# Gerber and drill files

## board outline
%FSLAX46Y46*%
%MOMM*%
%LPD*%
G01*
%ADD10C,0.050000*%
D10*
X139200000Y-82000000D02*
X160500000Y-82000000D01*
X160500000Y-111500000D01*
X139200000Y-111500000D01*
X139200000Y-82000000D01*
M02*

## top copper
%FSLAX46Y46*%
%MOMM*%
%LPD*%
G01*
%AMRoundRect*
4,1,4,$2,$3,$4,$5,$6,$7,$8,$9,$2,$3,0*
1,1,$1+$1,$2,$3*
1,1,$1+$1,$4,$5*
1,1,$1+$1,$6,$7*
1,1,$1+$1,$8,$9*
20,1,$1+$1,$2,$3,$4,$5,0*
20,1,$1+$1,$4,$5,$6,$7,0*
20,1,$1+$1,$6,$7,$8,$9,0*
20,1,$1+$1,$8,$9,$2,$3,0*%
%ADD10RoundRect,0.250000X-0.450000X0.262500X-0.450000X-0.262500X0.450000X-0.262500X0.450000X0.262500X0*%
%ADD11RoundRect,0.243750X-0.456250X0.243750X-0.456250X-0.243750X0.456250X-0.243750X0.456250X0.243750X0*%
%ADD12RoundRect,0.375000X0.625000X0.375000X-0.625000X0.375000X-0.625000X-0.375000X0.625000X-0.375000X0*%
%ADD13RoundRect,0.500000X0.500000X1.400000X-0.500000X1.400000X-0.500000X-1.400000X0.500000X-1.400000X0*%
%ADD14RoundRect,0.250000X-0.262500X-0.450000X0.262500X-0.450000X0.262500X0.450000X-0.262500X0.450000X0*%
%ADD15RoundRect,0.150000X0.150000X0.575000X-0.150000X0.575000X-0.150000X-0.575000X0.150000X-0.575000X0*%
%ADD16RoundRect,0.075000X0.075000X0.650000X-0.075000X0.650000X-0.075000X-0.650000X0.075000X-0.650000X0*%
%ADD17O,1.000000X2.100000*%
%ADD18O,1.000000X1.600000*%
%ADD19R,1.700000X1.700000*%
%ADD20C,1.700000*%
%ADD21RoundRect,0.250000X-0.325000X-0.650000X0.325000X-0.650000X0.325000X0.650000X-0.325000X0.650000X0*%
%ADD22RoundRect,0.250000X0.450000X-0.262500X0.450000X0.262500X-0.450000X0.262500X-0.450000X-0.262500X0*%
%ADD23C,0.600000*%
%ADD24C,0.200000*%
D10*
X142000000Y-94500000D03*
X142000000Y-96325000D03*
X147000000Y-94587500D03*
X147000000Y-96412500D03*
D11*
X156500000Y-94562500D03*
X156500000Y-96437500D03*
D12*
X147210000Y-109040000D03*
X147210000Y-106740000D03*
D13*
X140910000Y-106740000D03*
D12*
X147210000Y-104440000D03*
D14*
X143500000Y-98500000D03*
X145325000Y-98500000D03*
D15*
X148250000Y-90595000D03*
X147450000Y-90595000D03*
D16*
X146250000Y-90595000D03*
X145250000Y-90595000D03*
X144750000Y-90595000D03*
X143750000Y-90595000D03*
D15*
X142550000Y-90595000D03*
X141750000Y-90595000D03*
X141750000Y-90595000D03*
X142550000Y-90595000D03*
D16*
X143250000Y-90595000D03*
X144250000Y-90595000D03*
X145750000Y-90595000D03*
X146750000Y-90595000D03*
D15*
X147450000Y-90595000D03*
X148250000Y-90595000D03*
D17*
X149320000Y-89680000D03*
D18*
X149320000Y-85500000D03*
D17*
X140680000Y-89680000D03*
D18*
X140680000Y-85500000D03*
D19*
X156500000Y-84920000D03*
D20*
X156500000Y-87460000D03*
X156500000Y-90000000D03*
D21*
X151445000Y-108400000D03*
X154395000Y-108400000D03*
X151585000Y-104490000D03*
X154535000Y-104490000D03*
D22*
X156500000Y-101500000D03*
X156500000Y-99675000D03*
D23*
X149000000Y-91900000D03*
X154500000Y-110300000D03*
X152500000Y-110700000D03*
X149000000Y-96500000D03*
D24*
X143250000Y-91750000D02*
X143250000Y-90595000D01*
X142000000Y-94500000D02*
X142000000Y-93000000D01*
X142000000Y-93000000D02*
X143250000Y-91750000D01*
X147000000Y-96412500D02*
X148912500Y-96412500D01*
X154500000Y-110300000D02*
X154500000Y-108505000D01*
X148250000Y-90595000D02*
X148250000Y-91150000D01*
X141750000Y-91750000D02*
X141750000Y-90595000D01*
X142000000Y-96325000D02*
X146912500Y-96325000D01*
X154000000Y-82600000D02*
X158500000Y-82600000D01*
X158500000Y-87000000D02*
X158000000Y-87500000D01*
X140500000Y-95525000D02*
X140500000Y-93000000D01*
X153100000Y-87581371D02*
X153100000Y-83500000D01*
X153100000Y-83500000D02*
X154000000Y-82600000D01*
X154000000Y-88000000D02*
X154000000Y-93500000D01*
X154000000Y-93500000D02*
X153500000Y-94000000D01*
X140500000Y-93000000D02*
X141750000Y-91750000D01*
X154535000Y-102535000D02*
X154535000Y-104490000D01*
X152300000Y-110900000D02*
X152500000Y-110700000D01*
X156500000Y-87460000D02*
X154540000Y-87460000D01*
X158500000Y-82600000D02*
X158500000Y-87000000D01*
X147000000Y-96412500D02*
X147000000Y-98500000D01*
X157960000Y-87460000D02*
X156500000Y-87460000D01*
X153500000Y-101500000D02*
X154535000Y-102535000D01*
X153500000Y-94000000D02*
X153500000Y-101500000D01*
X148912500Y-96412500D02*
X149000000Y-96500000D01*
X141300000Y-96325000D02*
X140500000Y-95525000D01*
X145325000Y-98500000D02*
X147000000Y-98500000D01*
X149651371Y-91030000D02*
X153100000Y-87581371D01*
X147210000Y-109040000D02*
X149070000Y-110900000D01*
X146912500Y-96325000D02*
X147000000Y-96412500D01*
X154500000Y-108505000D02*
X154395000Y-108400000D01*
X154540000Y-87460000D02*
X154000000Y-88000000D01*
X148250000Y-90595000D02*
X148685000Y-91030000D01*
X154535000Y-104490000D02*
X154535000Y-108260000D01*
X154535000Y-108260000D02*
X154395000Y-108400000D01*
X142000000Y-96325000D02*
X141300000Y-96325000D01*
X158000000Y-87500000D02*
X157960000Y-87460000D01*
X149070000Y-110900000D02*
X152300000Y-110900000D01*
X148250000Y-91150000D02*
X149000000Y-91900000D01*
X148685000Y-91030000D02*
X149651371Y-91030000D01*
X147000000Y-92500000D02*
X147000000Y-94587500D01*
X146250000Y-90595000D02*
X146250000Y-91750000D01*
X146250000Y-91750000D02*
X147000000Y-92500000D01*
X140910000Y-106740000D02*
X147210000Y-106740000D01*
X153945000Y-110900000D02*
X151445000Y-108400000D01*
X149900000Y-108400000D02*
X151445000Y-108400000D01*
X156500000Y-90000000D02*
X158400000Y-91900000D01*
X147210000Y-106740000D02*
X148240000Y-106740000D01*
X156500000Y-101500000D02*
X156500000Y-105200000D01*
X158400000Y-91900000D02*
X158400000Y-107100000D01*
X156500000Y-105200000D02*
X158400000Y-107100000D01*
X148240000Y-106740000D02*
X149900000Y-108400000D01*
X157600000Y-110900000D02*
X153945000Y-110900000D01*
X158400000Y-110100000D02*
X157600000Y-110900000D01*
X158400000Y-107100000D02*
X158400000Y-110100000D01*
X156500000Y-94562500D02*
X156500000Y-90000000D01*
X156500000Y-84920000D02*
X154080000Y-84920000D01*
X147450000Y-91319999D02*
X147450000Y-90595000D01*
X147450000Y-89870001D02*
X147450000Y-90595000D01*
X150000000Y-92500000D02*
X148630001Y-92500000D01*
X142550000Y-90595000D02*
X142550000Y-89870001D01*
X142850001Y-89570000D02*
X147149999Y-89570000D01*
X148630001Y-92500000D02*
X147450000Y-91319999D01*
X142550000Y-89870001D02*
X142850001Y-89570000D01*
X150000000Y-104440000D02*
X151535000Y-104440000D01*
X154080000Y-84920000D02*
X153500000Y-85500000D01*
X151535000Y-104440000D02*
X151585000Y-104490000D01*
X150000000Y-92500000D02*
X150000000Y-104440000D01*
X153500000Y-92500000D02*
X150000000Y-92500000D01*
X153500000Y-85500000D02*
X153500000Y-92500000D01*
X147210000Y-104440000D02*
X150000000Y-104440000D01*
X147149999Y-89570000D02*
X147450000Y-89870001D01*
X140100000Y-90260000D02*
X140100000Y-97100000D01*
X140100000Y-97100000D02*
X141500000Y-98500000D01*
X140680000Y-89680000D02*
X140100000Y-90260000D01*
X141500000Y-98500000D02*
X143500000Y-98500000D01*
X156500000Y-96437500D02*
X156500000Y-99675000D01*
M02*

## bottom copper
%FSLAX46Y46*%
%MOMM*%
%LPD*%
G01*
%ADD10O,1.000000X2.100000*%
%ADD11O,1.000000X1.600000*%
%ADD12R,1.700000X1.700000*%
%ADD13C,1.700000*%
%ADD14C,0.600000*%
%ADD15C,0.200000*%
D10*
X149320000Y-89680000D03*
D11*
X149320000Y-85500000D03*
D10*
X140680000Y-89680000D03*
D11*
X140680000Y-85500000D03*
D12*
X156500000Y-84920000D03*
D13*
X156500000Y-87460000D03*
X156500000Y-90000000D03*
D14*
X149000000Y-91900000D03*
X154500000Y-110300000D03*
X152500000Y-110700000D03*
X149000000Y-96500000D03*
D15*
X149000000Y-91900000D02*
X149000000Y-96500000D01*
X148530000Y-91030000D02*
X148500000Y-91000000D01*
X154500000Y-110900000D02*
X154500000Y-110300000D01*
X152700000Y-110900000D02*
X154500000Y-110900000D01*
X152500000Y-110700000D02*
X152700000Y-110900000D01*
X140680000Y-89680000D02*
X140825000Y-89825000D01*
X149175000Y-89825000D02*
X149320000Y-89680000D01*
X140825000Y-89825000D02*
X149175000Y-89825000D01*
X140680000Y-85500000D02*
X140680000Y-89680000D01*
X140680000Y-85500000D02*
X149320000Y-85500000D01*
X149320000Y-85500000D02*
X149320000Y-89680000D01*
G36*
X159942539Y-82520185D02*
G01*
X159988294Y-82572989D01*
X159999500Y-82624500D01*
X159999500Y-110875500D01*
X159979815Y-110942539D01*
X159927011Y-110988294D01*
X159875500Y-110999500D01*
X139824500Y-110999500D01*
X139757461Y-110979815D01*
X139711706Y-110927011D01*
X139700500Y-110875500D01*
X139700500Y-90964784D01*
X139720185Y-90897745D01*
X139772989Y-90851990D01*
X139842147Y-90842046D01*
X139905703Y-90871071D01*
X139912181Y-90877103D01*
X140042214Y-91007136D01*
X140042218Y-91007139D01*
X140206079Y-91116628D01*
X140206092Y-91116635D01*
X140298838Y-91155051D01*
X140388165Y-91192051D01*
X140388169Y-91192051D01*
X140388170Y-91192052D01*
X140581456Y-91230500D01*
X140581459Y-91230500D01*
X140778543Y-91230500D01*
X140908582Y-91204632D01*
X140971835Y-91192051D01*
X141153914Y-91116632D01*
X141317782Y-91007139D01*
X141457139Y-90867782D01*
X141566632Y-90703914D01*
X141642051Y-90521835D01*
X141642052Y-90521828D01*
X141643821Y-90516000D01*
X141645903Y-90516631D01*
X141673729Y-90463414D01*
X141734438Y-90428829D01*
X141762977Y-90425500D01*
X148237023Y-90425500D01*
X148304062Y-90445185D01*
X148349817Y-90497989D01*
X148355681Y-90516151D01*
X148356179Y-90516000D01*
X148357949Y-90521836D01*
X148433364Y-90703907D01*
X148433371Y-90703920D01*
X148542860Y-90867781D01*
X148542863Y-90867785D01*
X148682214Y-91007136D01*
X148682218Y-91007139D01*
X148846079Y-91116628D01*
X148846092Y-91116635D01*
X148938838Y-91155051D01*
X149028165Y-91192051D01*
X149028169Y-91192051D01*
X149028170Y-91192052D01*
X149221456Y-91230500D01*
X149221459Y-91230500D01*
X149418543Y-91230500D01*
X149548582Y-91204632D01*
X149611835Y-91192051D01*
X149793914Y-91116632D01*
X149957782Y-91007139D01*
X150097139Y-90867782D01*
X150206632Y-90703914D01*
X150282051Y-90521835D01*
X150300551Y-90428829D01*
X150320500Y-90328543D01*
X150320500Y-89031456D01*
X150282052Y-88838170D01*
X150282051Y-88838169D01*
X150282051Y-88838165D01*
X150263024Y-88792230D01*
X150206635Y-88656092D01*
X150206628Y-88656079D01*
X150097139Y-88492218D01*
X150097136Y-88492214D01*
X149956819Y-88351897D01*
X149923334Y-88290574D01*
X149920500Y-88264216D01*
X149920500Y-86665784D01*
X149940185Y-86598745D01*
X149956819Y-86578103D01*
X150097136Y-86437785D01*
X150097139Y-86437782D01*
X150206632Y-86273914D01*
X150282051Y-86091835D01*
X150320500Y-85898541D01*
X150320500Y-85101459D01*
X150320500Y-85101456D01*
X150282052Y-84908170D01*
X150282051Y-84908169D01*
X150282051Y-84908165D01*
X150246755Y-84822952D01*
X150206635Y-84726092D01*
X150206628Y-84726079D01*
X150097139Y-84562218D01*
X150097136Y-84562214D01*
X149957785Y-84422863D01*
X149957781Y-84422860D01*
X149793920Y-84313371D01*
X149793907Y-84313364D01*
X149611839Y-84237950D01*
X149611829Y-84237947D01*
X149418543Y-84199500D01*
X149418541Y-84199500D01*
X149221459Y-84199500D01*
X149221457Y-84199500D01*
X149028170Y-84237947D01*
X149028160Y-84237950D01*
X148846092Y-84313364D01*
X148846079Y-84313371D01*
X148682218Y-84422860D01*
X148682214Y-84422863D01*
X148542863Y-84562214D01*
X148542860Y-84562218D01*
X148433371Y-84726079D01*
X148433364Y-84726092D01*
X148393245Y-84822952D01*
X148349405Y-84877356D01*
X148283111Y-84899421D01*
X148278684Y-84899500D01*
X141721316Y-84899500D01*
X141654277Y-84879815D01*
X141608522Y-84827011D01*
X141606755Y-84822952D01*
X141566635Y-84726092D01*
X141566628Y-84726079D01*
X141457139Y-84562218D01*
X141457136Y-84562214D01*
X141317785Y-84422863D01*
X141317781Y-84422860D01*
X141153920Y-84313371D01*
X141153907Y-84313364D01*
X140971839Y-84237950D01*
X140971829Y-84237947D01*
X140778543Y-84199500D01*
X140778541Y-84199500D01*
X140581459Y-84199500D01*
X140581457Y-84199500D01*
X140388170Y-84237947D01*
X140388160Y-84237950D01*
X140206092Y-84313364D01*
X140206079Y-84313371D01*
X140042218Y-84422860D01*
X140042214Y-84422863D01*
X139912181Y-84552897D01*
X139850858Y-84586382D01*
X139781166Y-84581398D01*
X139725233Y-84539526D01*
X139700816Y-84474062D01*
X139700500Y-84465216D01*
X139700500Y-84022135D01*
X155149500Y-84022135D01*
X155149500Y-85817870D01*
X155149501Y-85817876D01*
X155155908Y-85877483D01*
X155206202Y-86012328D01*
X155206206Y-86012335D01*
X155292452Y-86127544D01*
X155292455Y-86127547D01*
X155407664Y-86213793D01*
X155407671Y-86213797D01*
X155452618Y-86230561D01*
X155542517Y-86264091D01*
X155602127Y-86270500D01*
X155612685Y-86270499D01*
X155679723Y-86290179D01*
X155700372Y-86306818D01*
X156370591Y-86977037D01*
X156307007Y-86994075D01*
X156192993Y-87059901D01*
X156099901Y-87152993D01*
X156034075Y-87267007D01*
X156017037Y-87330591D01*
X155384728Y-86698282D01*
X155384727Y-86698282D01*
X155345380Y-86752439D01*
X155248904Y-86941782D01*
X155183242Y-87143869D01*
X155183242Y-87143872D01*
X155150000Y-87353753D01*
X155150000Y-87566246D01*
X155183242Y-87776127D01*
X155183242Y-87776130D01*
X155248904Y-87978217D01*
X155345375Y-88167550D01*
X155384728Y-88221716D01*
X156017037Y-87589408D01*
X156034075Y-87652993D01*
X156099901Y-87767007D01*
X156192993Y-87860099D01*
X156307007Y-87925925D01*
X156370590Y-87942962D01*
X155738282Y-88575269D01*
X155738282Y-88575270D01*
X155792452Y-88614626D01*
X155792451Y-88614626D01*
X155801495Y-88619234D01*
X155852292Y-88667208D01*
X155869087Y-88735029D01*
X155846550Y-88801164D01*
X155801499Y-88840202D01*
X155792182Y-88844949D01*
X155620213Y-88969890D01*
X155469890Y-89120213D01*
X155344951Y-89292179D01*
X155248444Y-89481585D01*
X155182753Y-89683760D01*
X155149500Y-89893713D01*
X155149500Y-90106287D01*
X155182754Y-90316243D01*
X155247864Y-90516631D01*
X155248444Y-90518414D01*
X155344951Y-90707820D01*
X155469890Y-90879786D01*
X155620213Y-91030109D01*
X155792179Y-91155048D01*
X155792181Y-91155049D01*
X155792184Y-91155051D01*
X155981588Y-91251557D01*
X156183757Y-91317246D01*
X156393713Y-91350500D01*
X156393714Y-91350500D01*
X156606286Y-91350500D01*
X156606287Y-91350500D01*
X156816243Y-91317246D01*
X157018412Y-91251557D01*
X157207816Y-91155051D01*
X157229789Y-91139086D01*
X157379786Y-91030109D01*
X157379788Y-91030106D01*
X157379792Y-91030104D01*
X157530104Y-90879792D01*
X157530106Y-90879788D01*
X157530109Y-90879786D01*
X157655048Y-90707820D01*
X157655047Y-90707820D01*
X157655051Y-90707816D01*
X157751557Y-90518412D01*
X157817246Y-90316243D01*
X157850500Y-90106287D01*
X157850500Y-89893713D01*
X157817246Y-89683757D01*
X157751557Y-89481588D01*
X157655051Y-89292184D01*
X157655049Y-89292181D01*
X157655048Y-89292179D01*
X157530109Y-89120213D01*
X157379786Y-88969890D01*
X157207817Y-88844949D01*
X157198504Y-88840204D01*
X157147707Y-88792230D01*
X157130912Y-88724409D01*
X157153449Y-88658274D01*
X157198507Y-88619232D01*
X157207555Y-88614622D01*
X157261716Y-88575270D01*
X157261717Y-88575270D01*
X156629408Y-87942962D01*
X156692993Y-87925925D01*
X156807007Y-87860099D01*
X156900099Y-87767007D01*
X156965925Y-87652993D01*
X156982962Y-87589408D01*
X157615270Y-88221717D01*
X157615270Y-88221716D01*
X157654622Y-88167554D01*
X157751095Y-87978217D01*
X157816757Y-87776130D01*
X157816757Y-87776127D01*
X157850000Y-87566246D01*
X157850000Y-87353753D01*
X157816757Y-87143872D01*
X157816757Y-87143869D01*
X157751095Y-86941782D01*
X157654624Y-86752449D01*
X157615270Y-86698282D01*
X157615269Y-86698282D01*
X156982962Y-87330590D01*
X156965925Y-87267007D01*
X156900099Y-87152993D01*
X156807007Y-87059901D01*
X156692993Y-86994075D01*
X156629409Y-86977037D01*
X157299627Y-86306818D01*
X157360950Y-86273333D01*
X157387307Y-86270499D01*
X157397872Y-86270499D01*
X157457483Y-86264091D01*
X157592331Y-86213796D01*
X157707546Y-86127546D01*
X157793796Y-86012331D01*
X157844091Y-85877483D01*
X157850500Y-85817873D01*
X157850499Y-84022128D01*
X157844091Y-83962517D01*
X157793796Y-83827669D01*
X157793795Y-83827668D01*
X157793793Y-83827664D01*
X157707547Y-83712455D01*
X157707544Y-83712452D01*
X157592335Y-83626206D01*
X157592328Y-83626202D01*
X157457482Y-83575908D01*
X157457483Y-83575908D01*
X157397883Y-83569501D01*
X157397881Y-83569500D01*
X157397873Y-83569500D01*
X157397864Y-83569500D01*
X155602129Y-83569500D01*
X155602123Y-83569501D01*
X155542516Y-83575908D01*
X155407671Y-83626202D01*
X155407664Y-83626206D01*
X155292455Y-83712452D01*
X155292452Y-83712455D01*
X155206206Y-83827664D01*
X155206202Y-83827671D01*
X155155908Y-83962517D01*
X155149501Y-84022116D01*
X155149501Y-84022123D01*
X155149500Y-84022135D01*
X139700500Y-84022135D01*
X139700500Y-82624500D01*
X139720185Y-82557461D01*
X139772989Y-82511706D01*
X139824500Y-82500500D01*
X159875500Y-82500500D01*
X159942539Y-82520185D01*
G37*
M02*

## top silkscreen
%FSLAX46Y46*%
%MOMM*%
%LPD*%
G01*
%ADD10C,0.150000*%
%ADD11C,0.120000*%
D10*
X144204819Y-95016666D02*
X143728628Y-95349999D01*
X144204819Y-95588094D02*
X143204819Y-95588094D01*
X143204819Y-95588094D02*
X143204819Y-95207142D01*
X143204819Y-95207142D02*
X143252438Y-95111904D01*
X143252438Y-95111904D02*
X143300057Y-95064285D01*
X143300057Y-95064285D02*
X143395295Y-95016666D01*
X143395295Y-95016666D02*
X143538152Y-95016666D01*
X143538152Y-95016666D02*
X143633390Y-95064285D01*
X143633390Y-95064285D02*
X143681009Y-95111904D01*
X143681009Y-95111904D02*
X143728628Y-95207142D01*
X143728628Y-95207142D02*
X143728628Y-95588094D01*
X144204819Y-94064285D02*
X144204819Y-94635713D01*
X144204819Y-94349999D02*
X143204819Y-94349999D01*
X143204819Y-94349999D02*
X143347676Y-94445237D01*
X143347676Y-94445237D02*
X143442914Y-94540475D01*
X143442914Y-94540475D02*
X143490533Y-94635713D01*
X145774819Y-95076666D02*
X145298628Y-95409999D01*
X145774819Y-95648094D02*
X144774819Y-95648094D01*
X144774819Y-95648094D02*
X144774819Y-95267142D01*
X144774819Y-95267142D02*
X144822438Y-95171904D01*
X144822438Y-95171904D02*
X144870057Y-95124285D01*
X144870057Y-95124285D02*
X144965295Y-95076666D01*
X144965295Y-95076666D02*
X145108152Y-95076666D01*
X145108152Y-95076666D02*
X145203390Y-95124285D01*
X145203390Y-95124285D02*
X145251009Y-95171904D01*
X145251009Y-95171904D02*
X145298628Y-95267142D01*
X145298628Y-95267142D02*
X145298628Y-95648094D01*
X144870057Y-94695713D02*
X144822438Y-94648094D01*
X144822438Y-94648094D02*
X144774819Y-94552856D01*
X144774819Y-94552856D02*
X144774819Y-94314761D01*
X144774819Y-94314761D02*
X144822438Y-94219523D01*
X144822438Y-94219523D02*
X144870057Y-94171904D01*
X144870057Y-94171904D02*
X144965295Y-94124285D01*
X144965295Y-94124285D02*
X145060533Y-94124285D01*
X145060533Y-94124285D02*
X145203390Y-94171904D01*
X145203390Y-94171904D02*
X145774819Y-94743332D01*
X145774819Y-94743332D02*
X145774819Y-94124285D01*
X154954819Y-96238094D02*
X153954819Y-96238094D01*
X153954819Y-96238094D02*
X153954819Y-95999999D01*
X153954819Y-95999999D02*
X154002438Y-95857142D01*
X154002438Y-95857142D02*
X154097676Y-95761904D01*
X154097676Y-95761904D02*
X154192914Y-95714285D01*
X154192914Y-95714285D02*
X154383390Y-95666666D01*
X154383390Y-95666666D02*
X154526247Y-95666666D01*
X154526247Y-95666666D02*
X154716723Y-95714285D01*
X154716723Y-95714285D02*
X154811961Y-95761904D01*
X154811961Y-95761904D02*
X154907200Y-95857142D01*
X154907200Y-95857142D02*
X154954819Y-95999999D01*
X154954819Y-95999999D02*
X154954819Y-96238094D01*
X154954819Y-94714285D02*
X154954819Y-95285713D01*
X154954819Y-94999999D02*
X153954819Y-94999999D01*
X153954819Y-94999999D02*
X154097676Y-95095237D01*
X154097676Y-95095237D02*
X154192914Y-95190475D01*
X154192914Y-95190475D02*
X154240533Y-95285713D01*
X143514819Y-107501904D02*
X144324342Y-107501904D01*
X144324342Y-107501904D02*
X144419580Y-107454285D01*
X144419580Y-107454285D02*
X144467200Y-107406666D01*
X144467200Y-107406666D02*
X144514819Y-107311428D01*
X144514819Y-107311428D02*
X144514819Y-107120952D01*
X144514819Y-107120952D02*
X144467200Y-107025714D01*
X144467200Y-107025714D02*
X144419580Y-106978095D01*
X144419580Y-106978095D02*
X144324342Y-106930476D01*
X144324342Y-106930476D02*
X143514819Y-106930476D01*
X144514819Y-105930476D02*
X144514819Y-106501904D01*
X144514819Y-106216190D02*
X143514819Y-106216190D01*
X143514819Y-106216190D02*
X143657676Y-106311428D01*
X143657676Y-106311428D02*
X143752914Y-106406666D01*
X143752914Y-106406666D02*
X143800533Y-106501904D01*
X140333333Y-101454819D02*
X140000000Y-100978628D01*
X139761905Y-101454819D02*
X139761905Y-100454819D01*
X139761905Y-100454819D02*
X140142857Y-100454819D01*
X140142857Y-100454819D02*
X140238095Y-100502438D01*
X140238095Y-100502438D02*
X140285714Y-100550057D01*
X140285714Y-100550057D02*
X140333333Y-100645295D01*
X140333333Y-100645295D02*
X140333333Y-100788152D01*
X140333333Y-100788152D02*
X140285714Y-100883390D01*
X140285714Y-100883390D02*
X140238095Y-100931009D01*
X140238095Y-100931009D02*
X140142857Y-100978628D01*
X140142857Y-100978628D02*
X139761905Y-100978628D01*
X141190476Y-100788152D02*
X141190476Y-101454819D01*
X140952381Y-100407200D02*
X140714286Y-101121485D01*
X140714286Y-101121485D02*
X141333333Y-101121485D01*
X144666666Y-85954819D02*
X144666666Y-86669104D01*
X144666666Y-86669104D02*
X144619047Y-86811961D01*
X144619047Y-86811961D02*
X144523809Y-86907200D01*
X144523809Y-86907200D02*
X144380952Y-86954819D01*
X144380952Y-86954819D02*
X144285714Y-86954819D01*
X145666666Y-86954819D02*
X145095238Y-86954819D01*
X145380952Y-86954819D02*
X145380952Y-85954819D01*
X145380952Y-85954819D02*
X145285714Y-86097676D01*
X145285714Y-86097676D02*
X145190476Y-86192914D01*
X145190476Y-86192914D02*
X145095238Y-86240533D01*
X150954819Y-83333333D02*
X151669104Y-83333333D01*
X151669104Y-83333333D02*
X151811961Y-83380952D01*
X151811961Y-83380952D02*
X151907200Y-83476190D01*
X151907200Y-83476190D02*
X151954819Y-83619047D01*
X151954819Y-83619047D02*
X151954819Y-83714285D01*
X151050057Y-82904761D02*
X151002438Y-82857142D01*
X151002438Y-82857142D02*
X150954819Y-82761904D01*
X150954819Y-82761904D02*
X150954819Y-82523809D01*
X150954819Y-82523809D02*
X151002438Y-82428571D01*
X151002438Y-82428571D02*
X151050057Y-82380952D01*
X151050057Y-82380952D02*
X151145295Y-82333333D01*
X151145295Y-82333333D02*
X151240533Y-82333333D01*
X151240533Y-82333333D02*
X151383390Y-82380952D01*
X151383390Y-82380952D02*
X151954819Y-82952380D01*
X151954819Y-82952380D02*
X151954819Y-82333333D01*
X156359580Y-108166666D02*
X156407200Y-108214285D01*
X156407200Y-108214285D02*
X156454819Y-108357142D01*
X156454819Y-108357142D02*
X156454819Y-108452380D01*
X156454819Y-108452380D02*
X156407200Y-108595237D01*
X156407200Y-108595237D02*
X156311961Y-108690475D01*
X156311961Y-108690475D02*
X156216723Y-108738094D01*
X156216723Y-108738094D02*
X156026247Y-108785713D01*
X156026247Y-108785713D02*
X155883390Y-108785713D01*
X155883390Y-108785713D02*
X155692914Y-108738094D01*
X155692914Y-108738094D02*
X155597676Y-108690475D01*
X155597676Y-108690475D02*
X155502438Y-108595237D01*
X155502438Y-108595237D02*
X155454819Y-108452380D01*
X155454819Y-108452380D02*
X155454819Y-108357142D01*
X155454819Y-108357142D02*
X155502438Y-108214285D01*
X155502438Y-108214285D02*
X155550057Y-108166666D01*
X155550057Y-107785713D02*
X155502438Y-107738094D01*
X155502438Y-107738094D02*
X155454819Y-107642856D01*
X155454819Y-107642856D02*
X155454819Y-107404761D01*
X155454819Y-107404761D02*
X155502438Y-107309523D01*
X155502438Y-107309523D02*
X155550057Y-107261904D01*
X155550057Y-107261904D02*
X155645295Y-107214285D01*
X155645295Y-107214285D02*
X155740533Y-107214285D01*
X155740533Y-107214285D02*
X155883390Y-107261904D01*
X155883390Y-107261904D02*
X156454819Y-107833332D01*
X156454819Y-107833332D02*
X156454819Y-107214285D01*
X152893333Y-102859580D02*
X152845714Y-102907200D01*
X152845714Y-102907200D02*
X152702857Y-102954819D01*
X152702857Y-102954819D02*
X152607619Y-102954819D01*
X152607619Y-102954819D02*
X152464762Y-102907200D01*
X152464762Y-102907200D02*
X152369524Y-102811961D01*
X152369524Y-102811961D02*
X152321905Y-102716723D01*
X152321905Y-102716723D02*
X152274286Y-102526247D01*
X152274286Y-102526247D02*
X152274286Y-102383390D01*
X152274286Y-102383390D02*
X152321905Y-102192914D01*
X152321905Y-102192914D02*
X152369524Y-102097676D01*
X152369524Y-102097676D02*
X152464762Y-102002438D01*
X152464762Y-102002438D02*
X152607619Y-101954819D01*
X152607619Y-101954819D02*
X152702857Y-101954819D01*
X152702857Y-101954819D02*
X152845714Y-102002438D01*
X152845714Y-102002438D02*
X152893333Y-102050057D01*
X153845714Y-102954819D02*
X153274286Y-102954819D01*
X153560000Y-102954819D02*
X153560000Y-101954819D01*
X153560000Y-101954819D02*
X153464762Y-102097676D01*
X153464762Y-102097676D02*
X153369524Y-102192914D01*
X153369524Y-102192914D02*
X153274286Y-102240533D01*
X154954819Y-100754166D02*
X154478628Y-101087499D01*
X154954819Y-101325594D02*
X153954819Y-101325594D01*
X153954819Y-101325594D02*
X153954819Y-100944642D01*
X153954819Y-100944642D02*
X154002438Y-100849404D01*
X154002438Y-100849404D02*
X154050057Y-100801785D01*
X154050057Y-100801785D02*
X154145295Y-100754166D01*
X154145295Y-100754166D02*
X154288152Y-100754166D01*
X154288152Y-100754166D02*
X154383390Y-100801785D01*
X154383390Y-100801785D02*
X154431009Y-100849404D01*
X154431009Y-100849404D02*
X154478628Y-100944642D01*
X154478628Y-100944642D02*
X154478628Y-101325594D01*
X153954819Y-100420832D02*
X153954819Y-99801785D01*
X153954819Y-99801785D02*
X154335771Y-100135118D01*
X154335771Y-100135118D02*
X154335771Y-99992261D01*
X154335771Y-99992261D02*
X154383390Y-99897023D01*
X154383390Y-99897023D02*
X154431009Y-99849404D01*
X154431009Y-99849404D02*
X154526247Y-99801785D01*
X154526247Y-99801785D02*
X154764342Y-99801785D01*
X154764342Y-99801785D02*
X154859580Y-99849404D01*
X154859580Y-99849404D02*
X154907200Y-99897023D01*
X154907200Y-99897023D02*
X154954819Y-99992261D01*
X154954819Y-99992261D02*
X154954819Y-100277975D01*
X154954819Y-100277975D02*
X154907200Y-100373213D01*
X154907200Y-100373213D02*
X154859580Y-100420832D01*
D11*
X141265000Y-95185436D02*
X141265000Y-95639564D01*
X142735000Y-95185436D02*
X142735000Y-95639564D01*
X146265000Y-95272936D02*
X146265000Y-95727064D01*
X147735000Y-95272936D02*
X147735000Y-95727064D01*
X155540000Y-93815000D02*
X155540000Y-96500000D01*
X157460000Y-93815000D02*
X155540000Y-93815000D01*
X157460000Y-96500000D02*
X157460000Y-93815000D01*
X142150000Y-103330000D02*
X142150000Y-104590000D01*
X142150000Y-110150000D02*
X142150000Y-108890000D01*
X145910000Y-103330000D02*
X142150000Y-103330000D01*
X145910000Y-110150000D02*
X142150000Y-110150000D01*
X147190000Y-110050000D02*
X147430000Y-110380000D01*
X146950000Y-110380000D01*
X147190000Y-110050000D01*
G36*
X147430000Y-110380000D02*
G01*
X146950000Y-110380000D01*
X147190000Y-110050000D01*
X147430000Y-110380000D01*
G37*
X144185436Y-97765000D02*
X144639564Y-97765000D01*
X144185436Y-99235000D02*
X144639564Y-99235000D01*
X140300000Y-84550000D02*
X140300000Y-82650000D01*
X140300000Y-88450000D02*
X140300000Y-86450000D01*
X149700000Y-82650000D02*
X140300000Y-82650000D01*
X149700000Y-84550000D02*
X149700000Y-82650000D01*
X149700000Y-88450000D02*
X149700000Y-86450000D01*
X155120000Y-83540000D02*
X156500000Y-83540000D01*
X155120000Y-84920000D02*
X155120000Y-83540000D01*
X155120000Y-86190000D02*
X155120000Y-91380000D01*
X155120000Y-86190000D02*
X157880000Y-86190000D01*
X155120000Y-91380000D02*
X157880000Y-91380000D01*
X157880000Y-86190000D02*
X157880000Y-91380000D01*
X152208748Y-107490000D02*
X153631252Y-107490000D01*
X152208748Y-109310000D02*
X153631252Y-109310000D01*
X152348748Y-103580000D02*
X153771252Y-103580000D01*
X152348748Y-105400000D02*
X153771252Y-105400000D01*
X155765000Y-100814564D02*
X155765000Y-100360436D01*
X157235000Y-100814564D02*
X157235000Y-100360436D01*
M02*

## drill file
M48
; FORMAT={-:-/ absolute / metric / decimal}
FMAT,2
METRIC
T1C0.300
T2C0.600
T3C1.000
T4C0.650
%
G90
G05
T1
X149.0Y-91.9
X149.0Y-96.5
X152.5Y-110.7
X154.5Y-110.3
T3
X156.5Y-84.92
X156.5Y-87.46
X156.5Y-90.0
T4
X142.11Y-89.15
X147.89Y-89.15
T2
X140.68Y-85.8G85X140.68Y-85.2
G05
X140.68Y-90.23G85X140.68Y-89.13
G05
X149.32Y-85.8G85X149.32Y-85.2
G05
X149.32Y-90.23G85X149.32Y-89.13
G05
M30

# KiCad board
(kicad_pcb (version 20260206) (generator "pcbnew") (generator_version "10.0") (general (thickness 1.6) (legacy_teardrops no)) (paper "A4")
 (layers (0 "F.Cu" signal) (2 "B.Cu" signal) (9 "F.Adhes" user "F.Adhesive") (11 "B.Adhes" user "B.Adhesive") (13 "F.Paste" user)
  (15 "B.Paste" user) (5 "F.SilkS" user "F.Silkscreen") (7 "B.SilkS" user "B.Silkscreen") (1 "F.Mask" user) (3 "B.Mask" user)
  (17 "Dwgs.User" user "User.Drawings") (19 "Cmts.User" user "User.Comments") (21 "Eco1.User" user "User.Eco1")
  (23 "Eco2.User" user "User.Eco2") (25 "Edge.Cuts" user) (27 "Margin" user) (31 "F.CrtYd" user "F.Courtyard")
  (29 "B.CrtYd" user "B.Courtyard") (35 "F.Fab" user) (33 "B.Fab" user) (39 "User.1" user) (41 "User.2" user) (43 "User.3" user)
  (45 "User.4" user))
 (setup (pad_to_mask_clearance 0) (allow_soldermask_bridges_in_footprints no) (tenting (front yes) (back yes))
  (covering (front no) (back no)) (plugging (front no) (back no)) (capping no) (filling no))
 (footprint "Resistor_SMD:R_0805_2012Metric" (layer "F.Cu") (at 142 95.4125 -90)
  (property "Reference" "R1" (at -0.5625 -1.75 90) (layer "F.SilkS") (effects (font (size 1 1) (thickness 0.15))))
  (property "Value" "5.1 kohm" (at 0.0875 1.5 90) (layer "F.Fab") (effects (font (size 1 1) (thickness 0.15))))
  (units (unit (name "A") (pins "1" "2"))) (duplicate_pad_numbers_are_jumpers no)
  (fp_line (start -0.227064 0.735) (end 0.227064 0.735) (stroke (width 0.12) (type solid)) (layer "F.SilkS"))
  (fp_line (start -0.227064 -0.735) (end 0.227064 -0.735) (stroke (width 0.12) (type solid)) (layer "F.SilkS"))
  (pad "1" smd roundrect (at -0.9125 0 270) (size 1.025 1.4) (layers "F.Cu" "F.Mask" "F.Paste") (roundrect_rratio 0.243902)
   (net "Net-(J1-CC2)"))
  (pad "2" smd roundrect (at 0.9125 0 270) (size 1.025 1.4) (layers "F.Cu" "F.Mask" "F.Paste") (roundrect_rratio 0.243902) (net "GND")))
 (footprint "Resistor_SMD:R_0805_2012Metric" (layer "F.Cu") (at 147 95.5 -90)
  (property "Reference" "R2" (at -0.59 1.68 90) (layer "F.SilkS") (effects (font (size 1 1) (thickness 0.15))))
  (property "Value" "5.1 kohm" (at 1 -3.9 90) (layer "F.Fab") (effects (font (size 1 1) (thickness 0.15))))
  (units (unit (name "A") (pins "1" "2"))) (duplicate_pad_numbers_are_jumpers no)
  (fp_line (start -0.227064 0.735) (end 0.227064 0.735) (stroke (width 0.12) (type solid)) (layer "F.SilkS"))
  (fp_line (start -0.227064 -0.735) (end 0.227064 -0.735) (stroke (width 0.12) (type solid)) (layer "F.SilkS"))
  (pad "1" smd roundrect (at -0.9125 0 270) (size 1.025 1.4) (layers "F.Cu" "F.Mask" "F.Paste") (roundrect_rratio 0.243902)
   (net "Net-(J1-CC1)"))
  (pad "2" smd roundrect (at 0.9125 0 270) (size 1.025 1.4) (layers "F.Cu" "F.Mask" "F.Paste") (roundrect_rratio 0.243902) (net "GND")))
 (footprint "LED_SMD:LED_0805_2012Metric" (layer "F.Cu") (at 156.5 95.5 -90)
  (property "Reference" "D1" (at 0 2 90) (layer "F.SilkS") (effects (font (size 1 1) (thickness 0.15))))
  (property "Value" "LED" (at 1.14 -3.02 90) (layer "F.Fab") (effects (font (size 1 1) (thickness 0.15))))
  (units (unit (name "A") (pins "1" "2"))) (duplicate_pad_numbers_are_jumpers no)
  (fp_line (start -1.685 0.96) (end 1 0.96) (stroke (width 0.12) (type solid)) (layer "F.SilkS"))
  (fp_line (start -1.685 -0.96) (end -1.685 0.96) (stroke (width 0.12) (type solid)) (layer "F.SilkS"))
  (fp_line (start 1 -0.96) (end -1.685 -0.96) (stroke (width 0.12) (type solid)) (layer "F.SilkS"))
  (pad "1" smd roundrect (at -0.9375 0 270) (size 0.975 1.4) (layers "F.Cu" "F.Mask" "F.Paste") (roundrect_rratio 0.25) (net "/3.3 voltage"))
  (pad "2" smd roundrect (at 0.9375 0 270) (size 0.975 1.4) (layers "F.Cu" "F.Mask" "F.Paste") (roundrect_rratio 0.25) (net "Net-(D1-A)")))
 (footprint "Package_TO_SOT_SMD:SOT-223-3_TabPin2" (layer "F.Cu") (at 144.06 106.74 180)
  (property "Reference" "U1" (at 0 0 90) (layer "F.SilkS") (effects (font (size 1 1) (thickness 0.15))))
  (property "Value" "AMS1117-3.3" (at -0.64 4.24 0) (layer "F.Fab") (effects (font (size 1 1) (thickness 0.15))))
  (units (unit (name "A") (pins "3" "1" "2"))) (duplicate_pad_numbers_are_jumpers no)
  (fp_line (start 1.91 3.41) (end 1.91 2.15) (stroke (width 0.12) (type solid)) (layer "F.SilkS"))
  (fp_line (start 1.91 -3.41) (end 1.91 -2.15) (stroke (width 0.12) (type solid)) (layer "F.SilkS"))
  (fp_line (start -1.85 3.41) (end 1.91 3.41) (stroke (width 0.12) (type solid)) (layer "F.SilkS"))
  (fp_line (start -1.85 -3.41) (end 1.91 -3.41) (stroke (width 0.12) (type solid)) (layer "F.SilkS"))
  (fp_poly
   (pts (xy -3.13 -3.31) (xy -3.37 -3.64) (xy -2.89 -3.64) (xy -3.13 -3.31)) (stroke (width 0.12) (type solid)) (fill yes) (layer "F.SilkS"))
  (pad "1" smd roundrect (at -3.15 -2.3 180) (size 2 1.5) (layers "F.Cu" "F.Mask" "F.Paste") (roundrect_rratio 0.25) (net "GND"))
  (pad "2" smd roundrect (at -3.15 0 180) (size 2 1.5) (layers "F.Cu" "F.Mask" "F.Paste") (roundrect_rratio 0.25) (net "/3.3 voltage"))
  (pad "2" smd roundrect (at 3.15 0 180) (size 2 3.8) (layers "F.Cu" "F.Mask" "F.Paste") (roundrect_rratio 0.25) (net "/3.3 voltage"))
  (pad "3" smd roundrect (at -3.15 2.3 180) (size 2 1.5) (layers "F.Cu" "F.Mask" "F.Paste") (roundrect_rratio 0.25) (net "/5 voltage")))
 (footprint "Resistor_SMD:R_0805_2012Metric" (layer "F.Cu") (at 144.4125 98.5)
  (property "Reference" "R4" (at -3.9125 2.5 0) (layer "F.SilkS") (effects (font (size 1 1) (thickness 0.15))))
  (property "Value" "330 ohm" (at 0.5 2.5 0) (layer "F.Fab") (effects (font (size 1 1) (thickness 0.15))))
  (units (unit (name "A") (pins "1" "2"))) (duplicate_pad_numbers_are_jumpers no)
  (fp_line (start -0.227064 -0.735) (end 0.227064 -0.735) (stroke (width 0.12) (type solid)) (layer "F.SilkS"))
  (fp_line (start -0.227064 0.735) (end 0.227064 0.735) (stroke (width 0.12) (type solid)) (layer "F.SilkS"))
  (pad "1" smd roundrect (at -0.9125 0) (size 1.025 1.4) (layers "F.Cu" "F.Mask" "F.Paste") (roundrect_rratio 0.243902)
   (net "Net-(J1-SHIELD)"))
  (pad "2" smd roundrect (at 0.9125 0) (size 1.025 1.4) (layers "F.Cu" "F.Mask" "F.Paste") (roundrect_rratio 0.243902) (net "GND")))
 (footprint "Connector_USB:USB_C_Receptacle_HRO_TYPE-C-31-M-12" (layer "F.Cu") (at 145 86.55 180)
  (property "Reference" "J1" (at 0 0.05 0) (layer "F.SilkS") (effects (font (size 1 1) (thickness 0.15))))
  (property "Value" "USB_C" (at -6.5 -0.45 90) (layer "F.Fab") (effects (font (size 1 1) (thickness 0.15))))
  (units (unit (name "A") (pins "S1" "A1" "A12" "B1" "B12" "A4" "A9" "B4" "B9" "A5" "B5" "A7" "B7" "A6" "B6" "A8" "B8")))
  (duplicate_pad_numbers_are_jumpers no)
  (fp_line (start 4.7 2) (end 4.7 3.9) (stroke (width 0.12) (type solid)) (layer "F.SilkS"))
  (fp_line (start 4.7 -1.9) (end 4.7 0.1) (stroke (width 0.12) (type solid)) (layer "F.SilkS"))
  (fp_line (start -4.7 3.9) (end 4.7 3.9) (stroke (width 0.12) (type solid)) (layer "F.SilkS"))
  (fp_line (start -4.7 2) (end -4.7 3.9) (stroke (width 0.12) (type solid)) (layer "F.SilkS"))
  (fp_line (start -4.7 -1.9) (end -4.7 0.1) (stroke (width 0.12) (type solid)) (layer "F.SilkS"))
  (pad "" np_thru_hole circle (at -2.89 -2.6 180) (size 0.65 0.65) (drill 0.65) (layers "*.Cu" "*.Mask"))
  (pad "" np_thru_hole circle (at 2.89 -2.6 180) (size 0.65 0.65) (drill 0.65) (layers "*.Cu" "*.Mask"))
  (pad "A1" smd roundrect (at -3.25 -4.045 180) (size 0.6 1.45) (layers "F.Cu" "F.Mask" "F.Paste") (roundrect_rratio 0.25) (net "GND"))
  (pad "A4" smd roundrect (at -2.45 -4.045 180) (size 0.6 1.45) (layers "F.Cu" "F.Mask" "F.Paste") (roundrect_rratio 0.25)
   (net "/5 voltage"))
  (pad "A5" smd roundrect (at -1.25 -4.045 180) (size 0.3 1.45) (layers "F.Cu" "F.Mask" "F.Paste") (roundrect_rratio 0.25)
   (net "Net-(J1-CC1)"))
  (pad "A6" smd roundrect (at -0.25 -4.045 180) (size 0.3 1.45) (layers "F.Cu" "F.Mask" "F.Paste") (roundrect_rratio 0.25)
   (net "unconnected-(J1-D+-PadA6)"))
  (pad "A7" smd roundrect (at 0.25 -4.045 180) (size 0.3 1.45) (layers "F.Cu" "F.Mask" "F.Paste") (roundrect_rratio 0.25)
   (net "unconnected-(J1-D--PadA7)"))
  (pad "A8" smd roundrect (at 1.25 -4.045 180) (size 0.3 1.45) (layers "F.Cu" "F.Mask" "F.Paste") (roundrect_rratio 0.25)
   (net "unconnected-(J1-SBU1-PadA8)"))
  (pad "A9" smd roundrect (at 2.45 -4.045 180) (size 0.6 1.45) (layers "F.Cu" "F.Mask" "F.Paste") (roundrect_rratio 0.25) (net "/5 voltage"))
  (pad "A12" smd roundrect (at 3.25 -4.045 180) (size 0.6 1.45) (layers "F.Cu" "F.Mask" "F.Paste") (roundrect_rratio 0.25) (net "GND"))
  (pad "B1" smd roundrect (at 3.25 -4.045 180) (size 0.6 1.45) (layers "F.Cu" "F.Mask" "F.Paste") (roundrect_rratio 0.25) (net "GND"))
  (pad "B4" smd roundrect (at 2.45 -4.045 180) (size 0.6 1.45) (layers "F.Cu" "F.Mask" "F.Paste") (roundrect_rratio 0.25) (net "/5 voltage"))
  (pad "B5" smd roundrect (at 1.75 -4.045 180) (size 0.3 1.45) (layers "F.Cu" "F.Mask" "F.Paste") (roundrect_rratio 0.25)
   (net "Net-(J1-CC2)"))
  (pad "B6" smd roundrect (at 0.75 -4.045 180) (size 0.3 1.45) (layers "F.Cu" "F.Mask" "F.Paste") (roundrect_rratio 0.25)
   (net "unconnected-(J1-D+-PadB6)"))
  (pad "B7" smd roundrect (at -0.75 -4.045 180) (size 0.3 1.45) (layers "F.Cu" "F.Mask" "F.Paste") (roundrect_rratio 0.25)
   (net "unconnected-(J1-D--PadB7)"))
  (pad "B8" smd roundrect (at -1.75 -4.045 180) (size 0.3 1.45) (layers "F.Cu" "F.Mask" "F.Paste") (roundrect_rratio 0.25)
   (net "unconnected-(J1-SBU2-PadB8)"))
  (pad "B9" smd roundrect (at -2.45 -4.045 180) (size 0.6 1.45) (layers "F.Cu" "F.Mask" "F.Paste") (roundrect_rratio 0.25)
   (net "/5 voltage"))
  (pad "B12" smd roundrect (at -3.25 -4.045 180) (size 0.6 1.45) (layers "F.Cu" "F.Mask" "F.Paste") (roundrect_rratio 0.25) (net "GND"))
  (pad "SH" thru_hole oval (at -4.32 -3.13 180) (size 1 2.1) (drill oval 0.6 1.7) (layers "*.Cu" "*.Mask") (remove_unused_layers no)
   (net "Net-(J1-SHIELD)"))
  (pad "SH" thru_hole oval (at -4.32 1.05 180) (size 1 1.6) (drill oval 0.6 1.2) (layers "*.Cu" "*.Mask") (remove_unused_layers no)
   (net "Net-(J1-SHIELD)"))
  (pad "SH" thru_hole oval (at 4.32 -3.13 180) (size 1 2.1) (drill oval 0.6 1.7) (layers "*.Cu" "*.Mask") (remove_unused_layers no)
   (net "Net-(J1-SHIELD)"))
  (pad "SH" thru_hole oval (at 4.32 1.05 180) (size 1 1.6) (drill oval 0.6 1.2) (layers "*.Cu" "*.Mask") (remove_unused_layers no)
   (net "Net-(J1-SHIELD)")))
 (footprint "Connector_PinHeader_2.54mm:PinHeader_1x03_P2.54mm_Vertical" (layer "F.Cu") (at 156.5 84.92)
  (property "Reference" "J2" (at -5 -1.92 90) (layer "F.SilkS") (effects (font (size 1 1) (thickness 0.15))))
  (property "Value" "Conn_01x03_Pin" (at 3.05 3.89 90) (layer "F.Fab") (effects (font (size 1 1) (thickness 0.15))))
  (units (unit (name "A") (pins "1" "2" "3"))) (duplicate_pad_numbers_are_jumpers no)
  (fp_line (start -1.38 -1.38) (end 0 -1.38) (stroke (width 0.12) (type solid)) (layer "F.SilkS"))
  (fp_line (start -1.38 0) (end -1.38 -1.38) (stroke (width 0.12) (type solid)) (layer "F.SilkS"))
  (fp_line (start -1.38 1.27) (end -1.38 6.46) (stroke (width 0.12) (type solid)) (layer "F.SilkS"))
  (fp_line (start -1.38 1.27) (end 1.38 1.27) (stroke (width 0.12) (type solid)) (layer "F.SilkS"))
  (fp_line (start -1.38 6.46) (end 1.38 6.46) (stroke (width 0.12) (type solid)) (layer "F.SilkS"))
  (fp_line (start 1.38 1.27) (end 1.38 6.46) (stroke (width 0.12) (type solid)) (layer "F.SilkS"))
  (pad "1" thru_hole rect (at 0 0) (size 1.7 1.7) (drill 1) (layers "*.Cu" "*.Mask") (remove_unused_layers no) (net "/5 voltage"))
  (pad "2" thru_hole circle (at 0 2.54) (size 1.7 1.7) (drill 1) (layers "*.Cu" "*.Mask") (remove_unused_layers no) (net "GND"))
  (pad "3" thru_hole circle (at 0 5.08) (size 1.7 1.7) (drill 1) (layers "*.Cu" "*.Mask") (remove_unused_layers no) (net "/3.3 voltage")))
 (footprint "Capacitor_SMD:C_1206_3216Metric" (layer "F.Cu") (at 152.92 108.4)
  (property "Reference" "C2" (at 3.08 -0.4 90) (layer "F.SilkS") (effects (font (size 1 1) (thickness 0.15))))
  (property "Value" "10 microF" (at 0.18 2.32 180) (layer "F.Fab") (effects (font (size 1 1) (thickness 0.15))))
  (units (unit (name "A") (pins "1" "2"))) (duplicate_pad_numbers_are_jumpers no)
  (fp_line (start -0.711252 -0.91) (end 0.711252 -0.91) (stroke (width 0.12) (type solid)) (layer "F.SilkS"))
  (fp_line (start -0.711252 0.91) (end 0.711252 0.91) (stroke (width 0.12) (type solid)) (layer "F.SilkS"))
  (pad "1" smd roundrect (at -1.475 0) (size 1.15 1.8) (layers "F.Cu" "F.Mask" "F.Paste") (roundrect_rratio 0.217391) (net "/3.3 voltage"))
  (pad "2" smd roundrect (at 1.475 0) (size 1.15 1.8) (layers "F.Cu" "F.Mask" "F.Paste") (roundrect_rratio 0.217391) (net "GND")))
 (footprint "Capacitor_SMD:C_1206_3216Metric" (layer "F.Cu") (at 153.06 104.49)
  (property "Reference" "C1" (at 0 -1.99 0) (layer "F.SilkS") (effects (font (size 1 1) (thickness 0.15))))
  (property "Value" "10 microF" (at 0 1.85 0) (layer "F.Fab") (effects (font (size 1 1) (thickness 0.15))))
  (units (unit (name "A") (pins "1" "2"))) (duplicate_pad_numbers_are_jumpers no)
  (fp_line (start -0.711252 -0.91) (end 0.711252 -0.91) (stroke (width 0.12) (type solid)) (layer "F.SilkS"))
  (fp_line (start -0.711252 0.91) (end 0.711252 0.91) (stroke (width 0.12) (type solid)) (layer "F.SilkS"))
  (pad "1" smd roundrect (at -1.475 0) (size 1.15 1.8) (layers "F.Cu" "F.Mask" "F.Paste") (roundrect_rratio 0.217391) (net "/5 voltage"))
  (pad "2" smd roundrect (at 1.475 0) (size 1.15 1.8) (layers "F.Cu" "F.Mask" "F.Paste") (roundrect_rratio 0.217391) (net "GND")))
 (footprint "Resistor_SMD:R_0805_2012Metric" (layer "F.Cu") (at 156.5 100.5875 90)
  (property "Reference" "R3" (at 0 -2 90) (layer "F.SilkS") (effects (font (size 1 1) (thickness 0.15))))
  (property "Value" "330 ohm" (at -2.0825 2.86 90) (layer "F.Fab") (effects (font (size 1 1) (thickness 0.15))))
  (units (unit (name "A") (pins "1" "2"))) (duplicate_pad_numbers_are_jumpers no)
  (fp_line (start -0.227064 -0.735) (end 0.227064 -0.735) (stroke (width 0.12) (type solid)) (layer "F.SilkS"))
  (fp_line (start -0.227064 0.735) (end 0.227064 0.735) (stroke (width 0.12) (type solid)) (layer "F.SilkS"))
  (pad "1" smd roundrect (at -0.9125 0 90) (size 1.025 1.4) (layers "F.Cu" "F.Mask" "F.Paste") (roundrect_rratio 0.243902)
   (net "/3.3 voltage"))
  (pad "2" smd roundrect (at 0.9125 0 90) (size 1.025 1.4) (layers "F.Cu" "F.Mask" "F.Paste") (roundrect_rratio 0.243902) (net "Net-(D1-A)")))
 (gr_rect (start 139.2 82) (end 160.5 111.5) (stroke (width 0.05) (type default)) (fill no) (layer "Edge.Cuts"))
 (segment (start 143.25 91.75) (end 143.25 90.595) (width 0.2) (layer "F.Cu") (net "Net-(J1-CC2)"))
 (segment (start 142 94.5) (end 142 93) (width 0.2) (layer "F.Cu") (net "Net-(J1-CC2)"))
 (segment (start 142 93) (end 143.25 91.75) (width 0.2) (layer "F.Cu") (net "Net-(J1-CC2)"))
 (segment (start 147 96.4125) (end 148.9125 96.4125) (width 0.2) (layer "F.Cu") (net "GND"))
 (segment (start 154.5 110.3) (end 154.5 108.505) (width 0.2) (layer "F.Cu") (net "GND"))
 (segment (start 148.25 90.595) (end 148.25 91.15) (width 0.2) (layer "F.Cu") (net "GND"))
 (segment (start 141.75 91.75) (end 141.75 90.595) (width 0.2) (layer "F.Cu") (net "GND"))
 (segment (start 142 96.325) (end 146.9125 96.325) (width 0.2) (layer "F.Cu") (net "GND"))
 (segment (start 154 82.6) (end 158.5 82.6) (width 0.2) (layer "F.Cu") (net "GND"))
 (segment (start 158.5 87) (end 158 87.5) (width 0.2) (layer "F.Cu") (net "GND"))
 (segment (start 140.5 95.525) (end 140.5 93) (width 0.2) (layer "F.Cu") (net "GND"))
 (segment (start 153.1 87.581371) (end 153.1 83.5) (width 0.2) (layer "F.Cu") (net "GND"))
 (segment (start 153.1 83.5) (end 154 82.6) (width 0.2) (layer "F.Cu") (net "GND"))
 (segment (start 154 88) (end 154 93.5) (width 0.2) (layer "F.Cu") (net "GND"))
 (segment (start 154 93.5) (end 153.5 94) (width 0.2) (layer "F.Cu") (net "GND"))
 (segment (start 140.5 93) (end 141.75 91.75) (width 0.2) (layer "F.Cu") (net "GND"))
 (segment (start 154.535 102.535) (end 154.535 104.49) (width 0.2) (layer "F.Cu") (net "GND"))
 (segment (start 152.3 110.9) (end 152.5 110.7) (width 0.2) (layer "F.Cu") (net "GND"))
 (segment (start 156.5 87.46) (end 154.54 87.46) (width 0.2) (layer "F.Cu") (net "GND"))
 (segment (start 158.5 82.6) (end 158.5 87) (width 0.2) (layer "F.Cu") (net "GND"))
 (segment (start 147 96.4125) (end 147 98.5) (width 0.2) (layer "F.Cu") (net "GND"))
 (segment (start 157.96 87.46) (end 156.5 87.46) (width 0.2) (layer "F.Cu") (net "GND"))
 (segment (start 153.5 101.5) (end 154.535 102.535) (width 0.2) (layer "F.Cu") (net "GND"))
 (segment (start 153.5 94) (end 153.5 101.5) (width 0.2) (layer "F.Cu") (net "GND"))
 (segment (start 148.9125 96.4125) (end 149 96.5) (width 0.2) (layer "F.Cu") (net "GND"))
 (segment (start 141.3 96.325) (end 140.5 95.525) (width 0.2) (layer "F.Cu") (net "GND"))
 (segment (start 145.325 98.5) (end 147 98.5) (width 0.2) (layer "F.Cu") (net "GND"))
 (segment (start 149.651371 91.03) (end 153.1 87.581371) (width 0.2) (layer "F.Cu") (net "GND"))
 (segment (start 147.21 109.04) (end 149.07 110.9) (width 0.2) (layer "F.Cu") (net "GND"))
 (segment (start 146.9125 96.325) (end 147 96.4125) (width 0.2) (layer "F.Cu") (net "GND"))
 (segment (start 154.5 108.505) (end 154.395 108.4) (width 0.2) (layer "F.Cu") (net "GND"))
 (segment (start 154.54 87.46) (end 154 88) (width 0.2) (layer "F.Cu") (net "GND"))
 (segment (start 148.25 90.595) (end 148.685 91.03) (width 0.2) (layer "F.Cu") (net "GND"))
 (segment (start 154.535 104.49) (end 154.535 108.26) (width 0.2) (layer "F.Cu") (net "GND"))
 (segment (start 154.535 108.26) (end 154.395 108.4) (width 0.2) (layer "F.Cu") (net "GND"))
 (segment (start 142 96.325) (end 141.3 96.325) (width 0.2) (layer "F.Cu") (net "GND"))
 (segment (start 158 87.5) (end 157.96 87.46) (width 0.2) (layer "F.Cu") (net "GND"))
 (segment (start 149.07 110.9) (end 152.3 110.9) (width 0.2) (layer "F.Cu") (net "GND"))
 (segment (start 148.25 91.15) (end 149 91.9) (width 0.2) (layer "F.Cu") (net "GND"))
 (segment (start 148.685 91.03) (end 149.651371 91.03) (width 0.2) (layer "F.Cu") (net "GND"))
 (via (at 149 91.9) (size 0.6) (drill 0.3) (layers "F.Cu" "B.Cu") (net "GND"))
 (via (at 154.5 110.3) (size 0.6) (drill 0.3) (layers "F.Cu" "B.Cu") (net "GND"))
 (via (at 152.5 110.7) (size 0.6) (drill 0.3) (layers "F.Cu" "B.Cu") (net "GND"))
 (via (at 149 96.5) (size 0.6) (drill 0.3) (layers "F.Cu" "B.Cu") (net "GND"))
 (segment (start 149 91.9) (end 149 96.5) (width 0.2) (layer "B.Cu") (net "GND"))
 (segment (start 148.53 91.03) (end 148.5 91) (width 0.2) (layer "B.Cu") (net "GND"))
 (segment (start 154.5 110.9) (end 154.5 110.3) (width 0.2) (layer "B.Cu") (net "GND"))
 (segment (start 152.7 110.9) (end 154.5 110.9) (width 0.2) (layer "B.Cu") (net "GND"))
 (segment (start 152.5 110.7) (end 152.7 110.9) (width 0.2) (layer "B.Cu") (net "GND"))
 (segment (start 147 92.5) (end 147 94.5875) (width 0.2) (layer "F.Cu") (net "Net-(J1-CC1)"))
 (segment (start 146.25 90.595) (end 146.25 91.75) (width 0.2) (layer "F.Cu") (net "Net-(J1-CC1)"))
 (segment (start 146.25 91.75) (end 147 92.5) (width 0.2) (layer "F.Cu") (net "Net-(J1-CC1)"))
 (segment (start 140.91 106.74) (end 147.21 106.74) (width 0.2) (layer "F.Cu") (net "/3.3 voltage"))
 (segment (start 153.945 110.9) (end 151.445 108.4) (width 0.2) (layer "F.Cu") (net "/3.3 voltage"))
 (segment (start 149.9 108.4) (end 151.445 108.4) (width 0.2) (layer "F.Cu") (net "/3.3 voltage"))
 (segment (start 156.5 90) (end 158.4 91.9) (width 0.2) (layer "F.Cu") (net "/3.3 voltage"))
 (segment (start 147.21 106.74) (end 148.24 106.74) (width 0.2) (layer "F.Cu") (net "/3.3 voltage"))
 (segment (start 156.5 101.5) (end 156.5 105.2) (width 0.2) (layer "F.Cu") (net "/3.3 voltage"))
 (segment (start 158.4 91.9) (end 158.4 107.1) (width 0.2) (layer "F.Cu") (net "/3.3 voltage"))
 (segment (start 156.5 105.2) (end 158.4 107.1) (width 0.2) (layer "F.Cu") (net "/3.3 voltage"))
 (segment (start 148.24 106.74) (end 149.9 108.4) (width 0.2) (layer "F.Cu") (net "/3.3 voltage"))
 (segment (start 157.6 110.9) (end 153.945 110.9) (width 0.2) (layer "F.Cu") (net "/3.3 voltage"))
 (segment (start 158.4 110.1) (end 157.6 110.9) (width 0.2) (layer "F.Cu") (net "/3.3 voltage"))
 (segment (start 158.4 107.1) (end 158.4 110.1) (width 0.2) (layer "F.Cu") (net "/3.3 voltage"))
 (segment (start 156.5 94.5625) (end 156.5 90) (width 0.2) (layer "F.Cu") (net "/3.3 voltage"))
 (segment (start 156.5 84.92) (end 154.08 84.92) (width 0.2) (layer "F.Cu") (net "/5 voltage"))
 (segment (start 147.45 91.319999) (end 147.45 90.595) (width 0.2) (layer "F.Cu") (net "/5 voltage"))
 (segment (start 147.45 89.870001) (end 147.45 90.595) (width 0.2) (layer "F.Cu") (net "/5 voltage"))
 (segment (start 150 92.5) (end 148.630001 92.5) (width 0.2) (layer "F.Cu") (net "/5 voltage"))
 (segment (start 142.55 90.595) (end 142.55 89.870001) (width 0.2) (layer "F.Cu") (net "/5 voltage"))
 (segment (start 142.850001 89.57) (end 147.149999 89.57) (width 0.2) (layer "F.Cu") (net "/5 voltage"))
 (segment (start 148.630001 92.5) (end 147.45 91.319999) (width 0.2) (layer "F.Cu") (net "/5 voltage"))
 (segment (start 142.55 89.870001) (end 142.850001 89.57) (width 0.2) (layer "F.Cu") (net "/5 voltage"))
 (segment (start 150 104.44) (end 151.535 104.44) (width 0.2) (layer "F.Cu") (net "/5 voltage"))
 (segment (start 154.08 84.92) (end 153.5 85.5) (width 0.2) (layer "F.Cu") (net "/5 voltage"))
 (segment (start 151.535 104.44) (end 151.585 104.49) (width 0.2) (layer "F.Cu") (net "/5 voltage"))
 (segment (start 150 92.5) (end 150 104.44) (width 0.2) (layer "F.Cu") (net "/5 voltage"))
 (segment (start 153.5 92.5) (end 150 92.5) (width 0.2) (layer "F.Cu") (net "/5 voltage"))
 (segment (start 153.5 85.5) (end 153.5 92.5) (width 0.2) (layer "F.Cu") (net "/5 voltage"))
 (segment (start 147.21 104.44) (end 150 104.44) (width 0.2) (layer "F.Cu") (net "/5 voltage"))
 (segment (start 147.149999 89.57) (end 147.45 89.870001) (width 0.2) (layer "F.Cu") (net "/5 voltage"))
 (segment (start 140.1 90.26) (end 140.1 97.1) (width 0.2) (layer "F.Cu") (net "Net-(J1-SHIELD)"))
 (segment (start 140.1 97.1) (end 141.5 98.5) (width 0.2) (layer "F.Cu") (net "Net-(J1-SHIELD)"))
 (segment (start 140.68 89.68) (end 140.1 90.26) (width 0.2) (layer "F.Cu") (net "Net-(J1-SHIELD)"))
 (segment (start 141.5 98.5) (end 143.5 98.5) (width 0.2) (layer "F.Cu") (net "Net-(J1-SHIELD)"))
 (segment (start 140.68 89.68) (end 140.825 89.825) (width 0.2) (layer "B.Cu") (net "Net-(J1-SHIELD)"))
 (segment (start 149.175 89.825) (end 149.32 89.68) (width 0.2) (layer "B.Cu") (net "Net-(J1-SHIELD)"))
 (segment (start 140.825 89.825) (end 149.175 89.825) (width 0.2) (layer "B.Cu") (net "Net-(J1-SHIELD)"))
 (segment (start 140.68 85.5) (end 140.68 89.68) (width 0.2) (layer "B.Cu") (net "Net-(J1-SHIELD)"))
 (segment (start 140.68 85.5) (end 149.32 85.5) (width 0.2) (layer "B.Cu") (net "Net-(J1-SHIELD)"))
 (segment (start 149.32 85.5) (end 149.32 89.68) (width 0.2) (layer "B.Cu") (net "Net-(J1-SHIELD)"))
 (segment (start 156.5 96.4375) (end 156.5 99.675) (width 0.2) (layer "F.Cu") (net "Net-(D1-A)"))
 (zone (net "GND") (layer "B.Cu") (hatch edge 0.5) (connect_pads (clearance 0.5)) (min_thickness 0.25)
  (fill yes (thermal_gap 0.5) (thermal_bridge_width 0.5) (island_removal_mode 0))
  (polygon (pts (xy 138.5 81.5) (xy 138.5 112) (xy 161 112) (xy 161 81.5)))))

